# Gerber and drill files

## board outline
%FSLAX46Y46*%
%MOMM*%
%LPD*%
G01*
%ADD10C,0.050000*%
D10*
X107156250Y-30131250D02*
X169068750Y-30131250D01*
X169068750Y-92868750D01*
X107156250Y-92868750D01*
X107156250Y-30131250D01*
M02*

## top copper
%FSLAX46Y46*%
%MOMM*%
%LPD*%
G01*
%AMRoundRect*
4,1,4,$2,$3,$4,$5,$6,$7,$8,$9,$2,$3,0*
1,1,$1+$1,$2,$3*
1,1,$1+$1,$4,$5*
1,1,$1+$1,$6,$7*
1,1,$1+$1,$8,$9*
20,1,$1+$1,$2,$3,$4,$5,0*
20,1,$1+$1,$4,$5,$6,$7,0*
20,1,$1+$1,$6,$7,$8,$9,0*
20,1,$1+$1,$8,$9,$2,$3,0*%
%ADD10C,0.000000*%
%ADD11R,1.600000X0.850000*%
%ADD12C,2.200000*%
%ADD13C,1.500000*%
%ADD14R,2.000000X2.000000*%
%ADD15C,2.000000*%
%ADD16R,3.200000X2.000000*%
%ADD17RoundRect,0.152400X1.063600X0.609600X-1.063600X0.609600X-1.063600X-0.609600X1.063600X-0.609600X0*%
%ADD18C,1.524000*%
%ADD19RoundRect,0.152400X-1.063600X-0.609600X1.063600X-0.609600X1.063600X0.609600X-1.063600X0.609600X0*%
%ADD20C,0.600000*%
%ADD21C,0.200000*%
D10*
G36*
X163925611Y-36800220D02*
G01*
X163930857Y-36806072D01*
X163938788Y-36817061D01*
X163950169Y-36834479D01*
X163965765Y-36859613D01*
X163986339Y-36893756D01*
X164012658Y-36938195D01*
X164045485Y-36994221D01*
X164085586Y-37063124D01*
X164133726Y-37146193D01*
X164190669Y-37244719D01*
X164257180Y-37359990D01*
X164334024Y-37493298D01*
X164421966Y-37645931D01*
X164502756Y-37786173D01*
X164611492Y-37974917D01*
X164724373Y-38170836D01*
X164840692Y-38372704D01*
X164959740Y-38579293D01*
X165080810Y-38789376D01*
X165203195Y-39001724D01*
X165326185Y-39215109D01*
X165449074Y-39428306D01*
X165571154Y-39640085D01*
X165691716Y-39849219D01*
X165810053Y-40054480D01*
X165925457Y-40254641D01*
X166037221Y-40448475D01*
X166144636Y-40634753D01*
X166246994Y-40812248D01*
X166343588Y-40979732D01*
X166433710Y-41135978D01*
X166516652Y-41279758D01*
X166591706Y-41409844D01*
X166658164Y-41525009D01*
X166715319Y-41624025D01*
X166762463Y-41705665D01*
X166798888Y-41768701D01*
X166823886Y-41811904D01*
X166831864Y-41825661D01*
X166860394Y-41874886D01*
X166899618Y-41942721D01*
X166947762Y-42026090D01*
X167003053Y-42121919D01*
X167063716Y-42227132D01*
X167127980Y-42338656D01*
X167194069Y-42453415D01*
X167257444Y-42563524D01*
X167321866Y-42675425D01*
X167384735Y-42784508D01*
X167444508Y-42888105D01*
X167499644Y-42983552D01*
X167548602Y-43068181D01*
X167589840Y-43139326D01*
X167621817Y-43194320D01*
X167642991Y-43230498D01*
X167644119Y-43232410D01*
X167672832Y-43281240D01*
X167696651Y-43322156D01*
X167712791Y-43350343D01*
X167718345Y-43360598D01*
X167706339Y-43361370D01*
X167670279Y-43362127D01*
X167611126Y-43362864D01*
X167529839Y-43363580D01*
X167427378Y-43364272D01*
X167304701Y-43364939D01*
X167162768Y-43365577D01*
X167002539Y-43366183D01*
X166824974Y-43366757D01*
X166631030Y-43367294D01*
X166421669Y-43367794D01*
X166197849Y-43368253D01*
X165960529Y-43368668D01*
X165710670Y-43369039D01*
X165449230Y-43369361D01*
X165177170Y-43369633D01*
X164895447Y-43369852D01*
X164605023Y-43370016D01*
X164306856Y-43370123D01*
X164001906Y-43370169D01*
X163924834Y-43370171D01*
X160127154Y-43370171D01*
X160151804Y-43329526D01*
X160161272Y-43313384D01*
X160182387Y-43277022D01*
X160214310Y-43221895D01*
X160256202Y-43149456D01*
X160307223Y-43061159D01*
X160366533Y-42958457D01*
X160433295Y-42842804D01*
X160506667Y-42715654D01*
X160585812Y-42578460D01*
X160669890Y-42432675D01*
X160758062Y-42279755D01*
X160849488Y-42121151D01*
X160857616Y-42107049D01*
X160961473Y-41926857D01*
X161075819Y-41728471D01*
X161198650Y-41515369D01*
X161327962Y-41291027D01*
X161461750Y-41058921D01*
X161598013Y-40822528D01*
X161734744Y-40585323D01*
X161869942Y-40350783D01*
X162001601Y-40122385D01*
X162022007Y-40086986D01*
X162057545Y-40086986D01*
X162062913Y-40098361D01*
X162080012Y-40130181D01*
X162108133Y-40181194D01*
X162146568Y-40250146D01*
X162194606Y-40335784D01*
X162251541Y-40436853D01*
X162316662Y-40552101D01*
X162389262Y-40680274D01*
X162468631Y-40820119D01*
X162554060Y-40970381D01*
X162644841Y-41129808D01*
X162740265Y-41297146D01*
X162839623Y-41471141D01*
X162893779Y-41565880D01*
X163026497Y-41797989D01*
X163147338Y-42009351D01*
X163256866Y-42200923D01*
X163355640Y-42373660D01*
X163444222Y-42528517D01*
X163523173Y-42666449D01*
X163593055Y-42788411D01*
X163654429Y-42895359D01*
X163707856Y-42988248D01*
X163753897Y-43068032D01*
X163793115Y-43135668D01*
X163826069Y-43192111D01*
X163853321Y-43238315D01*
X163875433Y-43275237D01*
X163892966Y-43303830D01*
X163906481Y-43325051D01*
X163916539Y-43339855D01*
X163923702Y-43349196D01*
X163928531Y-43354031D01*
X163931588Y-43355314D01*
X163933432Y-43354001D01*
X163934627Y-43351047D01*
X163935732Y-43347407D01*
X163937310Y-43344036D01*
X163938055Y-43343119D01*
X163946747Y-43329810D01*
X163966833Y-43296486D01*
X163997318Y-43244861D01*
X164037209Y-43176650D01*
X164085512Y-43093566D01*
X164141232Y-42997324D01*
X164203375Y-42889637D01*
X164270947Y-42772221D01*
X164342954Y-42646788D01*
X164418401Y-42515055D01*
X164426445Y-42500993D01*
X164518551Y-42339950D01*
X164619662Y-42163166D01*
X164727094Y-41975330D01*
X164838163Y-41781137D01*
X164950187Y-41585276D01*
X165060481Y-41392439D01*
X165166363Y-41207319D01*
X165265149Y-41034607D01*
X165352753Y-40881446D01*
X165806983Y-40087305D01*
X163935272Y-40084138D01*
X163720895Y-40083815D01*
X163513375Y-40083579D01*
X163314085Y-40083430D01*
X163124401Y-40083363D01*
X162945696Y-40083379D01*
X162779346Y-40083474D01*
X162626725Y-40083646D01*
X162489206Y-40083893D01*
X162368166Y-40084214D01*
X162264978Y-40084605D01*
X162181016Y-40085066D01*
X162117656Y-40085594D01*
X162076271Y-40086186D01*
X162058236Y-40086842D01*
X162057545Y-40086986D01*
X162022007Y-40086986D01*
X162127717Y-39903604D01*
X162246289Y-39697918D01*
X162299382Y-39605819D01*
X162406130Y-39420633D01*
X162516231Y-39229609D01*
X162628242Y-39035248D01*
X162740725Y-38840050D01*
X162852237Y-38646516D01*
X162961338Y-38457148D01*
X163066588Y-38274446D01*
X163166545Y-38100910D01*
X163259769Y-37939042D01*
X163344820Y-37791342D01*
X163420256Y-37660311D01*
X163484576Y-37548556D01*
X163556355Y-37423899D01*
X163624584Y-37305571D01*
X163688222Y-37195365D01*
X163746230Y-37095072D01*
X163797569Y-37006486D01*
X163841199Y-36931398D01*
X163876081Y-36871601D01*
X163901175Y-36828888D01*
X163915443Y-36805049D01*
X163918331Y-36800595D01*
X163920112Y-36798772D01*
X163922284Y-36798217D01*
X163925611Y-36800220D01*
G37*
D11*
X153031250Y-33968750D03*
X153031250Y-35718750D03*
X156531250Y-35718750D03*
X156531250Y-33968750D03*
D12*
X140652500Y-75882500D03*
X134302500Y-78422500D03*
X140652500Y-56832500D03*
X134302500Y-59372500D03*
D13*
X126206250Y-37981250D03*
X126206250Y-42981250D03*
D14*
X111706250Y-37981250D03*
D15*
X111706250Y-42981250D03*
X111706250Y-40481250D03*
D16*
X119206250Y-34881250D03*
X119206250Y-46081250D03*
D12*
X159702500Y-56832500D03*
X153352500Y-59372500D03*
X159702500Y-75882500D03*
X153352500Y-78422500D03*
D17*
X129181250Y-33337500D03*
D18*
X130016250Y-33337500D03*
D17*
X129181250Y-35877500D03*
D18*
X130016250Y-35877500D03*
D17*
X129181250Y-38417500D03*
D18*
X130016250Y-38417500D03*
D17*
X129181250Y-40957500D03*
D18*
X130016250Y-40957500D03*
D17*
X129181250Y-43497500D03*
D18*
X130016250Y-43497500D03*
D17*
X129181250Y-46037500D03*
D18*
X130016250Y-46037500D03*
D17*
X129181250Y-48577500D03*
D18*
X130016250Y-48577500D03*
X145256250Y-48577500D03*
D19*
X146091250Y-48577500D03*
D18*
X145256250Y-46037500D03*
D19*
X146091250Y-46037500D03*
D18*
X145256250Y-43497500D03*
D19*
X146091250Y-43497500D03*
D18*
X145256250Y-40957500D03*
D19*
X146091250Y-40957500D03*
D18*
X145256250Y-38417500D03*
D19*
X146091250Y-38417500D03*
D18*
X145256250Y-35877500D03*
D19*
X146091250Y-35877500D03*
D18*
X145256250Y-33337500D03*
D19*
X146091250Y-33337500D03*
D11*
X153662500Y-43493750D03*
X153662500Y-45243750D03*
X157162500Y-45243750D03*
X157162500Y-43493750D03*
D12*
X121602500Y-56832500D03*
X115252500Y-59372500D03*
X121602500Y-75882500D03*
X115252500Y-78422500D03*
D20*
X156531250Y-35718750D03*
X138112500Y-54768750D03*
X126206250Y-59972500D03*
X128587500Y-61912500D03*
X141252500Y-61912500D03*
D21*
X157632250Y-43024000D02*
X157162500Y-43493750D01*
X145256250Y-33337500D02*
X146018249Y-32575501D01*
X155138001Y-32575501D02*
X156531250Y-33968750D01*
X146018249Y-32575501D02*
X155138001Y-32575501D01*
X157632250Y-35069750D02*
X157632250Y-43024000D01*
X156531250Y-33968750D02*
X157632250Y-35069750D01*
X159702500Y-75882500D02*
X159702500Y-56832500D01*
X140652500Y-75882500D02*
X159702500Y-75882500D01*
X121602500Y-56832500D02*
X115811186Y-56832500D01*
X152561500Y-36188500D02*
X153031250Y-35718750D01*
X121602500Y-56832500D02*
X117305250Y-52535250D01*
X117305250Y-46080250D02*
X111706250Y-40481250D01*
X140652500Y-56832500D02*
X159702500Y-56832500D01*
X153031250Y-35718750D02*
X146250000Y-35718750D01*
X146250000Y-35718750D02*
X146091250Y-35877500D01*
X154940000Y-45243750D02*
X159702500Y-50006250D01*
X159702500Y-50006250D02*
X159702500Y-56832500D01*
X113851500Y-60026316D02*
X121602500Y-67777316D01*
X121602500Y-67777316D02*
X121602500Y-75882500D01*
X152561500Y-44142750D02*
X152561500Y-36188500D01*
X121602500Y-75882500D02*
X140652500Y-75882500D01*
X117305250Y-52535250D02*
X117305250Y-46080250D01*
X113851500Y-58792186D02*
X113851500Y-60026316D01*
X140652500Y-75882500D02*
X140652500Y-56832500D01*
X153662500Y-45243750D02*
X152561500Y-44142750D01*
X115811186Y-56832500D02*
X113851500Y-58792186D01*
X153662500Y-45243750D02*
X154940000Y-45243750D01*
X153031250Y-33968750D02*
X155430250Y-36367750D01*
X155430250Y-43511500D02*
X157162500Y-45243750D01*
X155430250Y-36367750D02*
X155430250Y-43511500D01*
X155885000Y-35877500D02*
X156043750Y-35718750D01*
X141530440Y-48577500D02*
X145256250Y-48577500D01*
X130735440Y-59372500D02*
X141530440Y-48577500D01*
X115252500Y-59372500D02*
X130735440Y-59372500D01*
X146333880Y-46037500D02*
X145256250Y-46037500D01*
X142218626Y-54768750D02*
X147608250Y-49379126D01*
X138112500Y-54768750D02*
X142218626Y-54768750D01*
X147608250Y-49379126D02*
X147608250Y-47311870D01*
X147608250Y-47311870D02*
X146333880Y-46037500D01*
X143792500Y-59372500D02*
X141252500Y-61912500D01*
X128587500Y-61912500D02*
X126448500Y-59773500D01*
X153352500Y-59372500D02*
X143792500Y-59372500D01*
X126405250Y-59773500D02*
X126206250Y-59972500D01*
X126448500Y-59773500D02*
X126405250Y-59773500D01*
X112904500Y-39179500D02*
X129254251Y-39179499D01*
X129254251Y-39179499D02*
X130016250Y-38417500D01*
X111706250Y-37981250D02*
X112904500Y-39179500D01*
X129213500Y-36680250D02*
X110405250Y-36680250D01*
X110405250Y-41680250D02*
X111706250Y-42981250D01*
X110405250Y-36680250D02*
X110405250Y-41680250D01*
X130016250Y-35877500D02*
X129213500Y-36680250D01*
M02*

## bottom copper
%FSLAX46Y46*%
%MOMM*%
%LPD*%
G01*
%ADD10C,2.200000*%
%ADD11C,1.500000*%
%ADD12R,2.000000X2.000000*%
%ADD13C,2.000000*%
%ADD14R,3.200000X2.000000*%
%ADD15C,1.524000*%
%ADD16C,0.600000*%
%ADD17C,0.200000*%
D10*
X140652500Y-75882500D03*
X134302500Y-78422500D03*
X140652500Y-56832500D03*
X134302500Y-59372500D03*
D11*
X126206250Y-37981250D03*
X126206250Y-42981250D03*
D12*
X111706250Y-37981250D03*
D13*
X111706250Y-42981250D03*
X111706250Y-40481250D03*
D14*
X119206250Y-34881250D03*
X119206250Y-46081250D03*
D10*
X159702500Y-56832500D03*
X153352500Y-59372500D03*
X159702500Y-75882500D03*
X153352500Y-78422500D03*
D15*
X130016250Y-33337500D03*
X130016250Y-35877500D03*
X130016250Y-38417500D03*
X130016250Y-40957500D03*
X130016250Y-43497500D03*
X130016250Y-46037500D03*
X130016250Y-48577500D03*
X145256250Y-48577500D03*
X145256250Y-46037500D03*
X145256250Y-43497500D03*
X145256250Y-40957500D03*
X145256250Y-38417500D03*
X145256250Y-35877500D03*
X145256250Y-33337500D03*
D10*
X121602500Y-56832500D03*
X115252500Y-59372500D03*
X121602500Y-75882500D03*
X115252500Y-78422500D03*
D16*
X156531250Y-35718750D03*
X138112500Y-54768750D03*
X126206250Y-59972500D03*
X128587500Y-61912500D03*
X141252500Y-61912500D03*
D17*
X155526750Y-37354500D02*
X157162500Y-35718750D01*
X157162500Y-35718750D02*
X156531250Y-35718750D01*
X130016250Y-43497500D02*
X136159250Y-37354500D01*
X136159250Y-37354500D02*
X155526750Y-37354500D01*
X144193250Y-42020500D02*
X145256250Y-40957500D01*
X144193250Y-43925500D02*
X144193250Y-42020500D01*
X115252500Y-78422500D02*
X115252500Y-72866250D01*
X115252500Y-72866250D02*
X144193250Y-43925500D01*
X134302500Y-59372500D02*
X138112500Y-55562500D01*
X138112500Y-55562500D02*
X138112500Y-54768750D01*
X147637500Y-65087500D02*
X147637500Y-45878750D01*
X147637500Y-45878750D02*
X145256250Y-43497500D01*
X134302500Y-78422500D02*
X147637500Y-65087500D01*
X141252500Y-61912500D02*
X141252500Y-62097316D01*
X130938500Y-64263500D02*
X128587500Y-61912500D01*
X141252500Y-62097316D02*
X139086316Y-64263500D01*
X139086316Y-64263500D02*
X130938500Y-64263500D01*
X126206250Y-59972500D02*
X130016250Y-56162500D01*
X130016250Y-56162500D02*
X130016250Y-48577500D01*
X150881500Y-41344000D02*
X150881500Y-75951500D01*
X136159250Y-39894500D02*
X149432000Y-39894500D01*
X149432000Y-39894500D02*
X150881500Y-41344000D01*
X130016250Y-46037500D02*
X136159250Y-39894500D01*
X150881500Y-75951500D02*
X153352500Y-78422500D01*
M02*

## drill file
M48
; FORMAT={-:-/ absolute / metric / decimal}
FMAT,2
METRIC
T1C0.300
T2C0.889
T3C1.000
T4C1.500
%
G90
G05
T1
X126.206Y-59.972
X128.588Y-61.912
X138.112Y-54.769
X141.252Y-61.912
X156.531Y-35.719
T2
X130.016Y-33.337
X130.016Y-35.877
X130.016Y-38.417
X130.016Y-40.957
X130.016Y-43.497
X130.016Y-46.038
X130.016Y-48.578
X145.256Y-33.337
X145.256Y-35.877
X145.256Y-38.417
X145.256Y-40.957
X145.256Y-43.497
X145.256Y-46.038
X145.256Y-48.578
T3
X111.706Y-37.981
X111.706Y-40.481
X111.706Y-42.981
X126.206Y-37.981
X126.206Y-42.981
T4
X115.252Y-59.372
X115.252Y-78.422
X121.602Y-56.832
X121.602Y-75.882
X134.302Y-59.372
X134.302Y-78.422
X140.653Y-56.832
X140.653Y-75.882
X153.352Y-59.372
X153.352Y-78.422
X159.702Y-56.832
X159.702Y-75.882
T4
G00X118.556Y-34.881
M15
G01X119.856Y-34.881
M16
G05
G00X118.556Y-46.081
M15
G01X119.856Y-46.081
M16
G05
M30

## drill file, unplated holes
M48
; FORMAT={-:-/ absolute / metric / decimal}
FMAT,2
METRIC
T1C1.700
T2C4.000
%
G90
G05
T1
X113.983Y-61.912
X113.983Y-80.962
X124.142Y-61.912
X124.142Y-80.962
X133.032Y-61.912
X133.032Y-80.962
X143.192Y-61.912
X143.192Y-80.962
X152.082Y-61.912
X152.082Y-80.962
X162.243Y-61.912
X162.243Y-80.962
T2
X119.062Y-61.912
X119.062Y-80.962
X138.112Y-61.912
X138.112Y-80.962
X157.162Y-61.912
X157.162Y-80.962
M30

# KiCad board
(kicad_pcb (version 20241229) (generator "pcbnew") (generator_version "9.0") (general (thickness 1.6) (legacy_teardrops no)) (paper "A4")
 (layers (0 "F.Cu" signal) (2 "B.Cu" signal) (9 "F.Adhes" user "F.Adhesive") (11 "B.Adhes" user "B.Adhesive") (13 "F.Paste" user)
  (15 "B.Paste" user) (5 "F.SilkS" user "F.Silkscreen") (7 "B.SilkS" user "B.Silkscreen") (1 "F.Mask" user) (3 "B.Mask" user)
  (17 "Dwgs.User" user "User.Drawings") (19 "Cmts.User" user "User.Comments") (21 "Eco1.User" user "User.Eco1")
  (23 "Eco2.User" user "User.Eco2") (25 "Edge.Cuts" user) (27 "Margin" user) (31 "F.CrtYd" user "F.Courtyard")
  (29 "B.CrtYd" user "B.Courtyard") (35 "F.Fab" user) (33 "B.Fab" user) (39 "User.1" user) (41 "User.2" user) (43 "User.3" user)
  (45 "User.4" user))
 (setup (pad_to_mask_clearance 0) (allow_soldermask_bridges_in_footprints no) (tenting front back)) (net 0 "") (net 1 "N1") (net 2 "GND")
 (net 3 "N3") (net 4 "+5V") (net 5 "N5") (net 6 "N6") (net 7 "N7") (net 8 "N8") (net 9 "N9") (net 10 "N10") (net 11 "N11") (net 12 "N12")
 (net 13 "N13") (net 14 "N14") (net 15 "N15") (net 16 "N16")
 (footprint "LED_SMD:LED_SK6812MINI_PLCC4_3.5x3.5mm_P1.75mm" (layer "F.Cu") (at 154.78125 34.84375)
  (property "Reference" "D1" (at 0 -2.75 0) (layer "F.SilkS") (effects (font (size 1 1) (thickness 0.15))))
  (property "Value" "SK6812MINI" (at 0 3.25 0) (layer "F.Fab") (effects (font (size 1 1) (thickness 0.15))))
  (pad "1" smd rect (at -1.75 -0.875) (size 1.6 0.85) (layers "F.Cu" "F.Mask" "F.Paste") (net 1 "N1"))
  (pad "2" smd rect (at -1.75 0.875) (size 1.6 0.85) (layers "F.Cu" "F.Mask" "F.Paste") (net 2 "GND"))
  (pad "3" smd rect (at 1.75 0.875) (size 1.6 0.85) (layers "F.Cu" "F.Mask" "F.Paste") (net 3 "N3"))
  (pad "4" smd rect (at 1.75 -0.875) (size 1.6 0.85) (layers "F.Cu" "F.Mask" "F.Paste") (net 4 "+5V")))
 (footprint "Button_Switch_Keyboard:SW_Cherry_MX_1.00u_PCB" (layer "F.Cu") (at 140.6525 75.8825)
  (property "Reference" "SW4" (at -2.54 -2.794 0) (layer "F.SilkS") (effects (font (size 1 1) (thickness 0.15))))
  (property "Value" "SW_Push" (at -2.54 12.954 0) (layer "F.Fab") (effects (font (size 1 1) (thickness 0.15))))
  (pad "" np_thru_hole circle (at -7.62 5.08) (size 1.7 1.7) (drill 1.7) (layers "*.Cu" "*.Mask"))
  (pad "" np_thru_hole circle (at -2.54 5.08) (size 4 4) (drill 4) (layers "*.Cu" "*.Mask"))
  (pad "" np_thru_hole circle (at 2.54 5.08) (size 1.7 1.7) (drill 1.7) (layers "*.Cu" "*.Mask"))
  (pad "1" thru_hole circle (at 0 0) (size 2.2 2.2) (drill 1.5) (layers "*.Cu" "*.Mask") (remove_unused_layers no) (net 2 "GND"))
  (pad "2" thru_hole circle (at -6.35 2.54) (size 2.2 2.2) (drill 1.5) (layers "*.Cu" "*.Mask") (remove_unused_layers no) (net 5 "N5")))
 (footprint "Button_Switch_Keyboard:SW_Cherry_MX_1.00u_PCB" (layer "F.Cu") (at 140.6525 56.8325)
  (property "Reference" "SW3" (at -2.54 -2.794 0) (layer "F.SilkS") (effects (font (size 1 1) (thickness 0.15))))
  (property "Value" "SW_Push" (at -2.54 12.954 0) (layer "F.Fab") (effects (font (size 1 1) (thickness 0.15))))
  (pad "" np_thru_hole circle (at -7.62 5.08) (size 1.7 1.7) (drill 1.7) (layers "*.Cu" "*.Mask"))
  (pad "" np_thru_hole circle (at -2.54 5.08) (size 4 4) (drill 4) (layers "*.Cu" "*.Mask"))
  (pad "" np_thru_hole circle (at 2.54 5.08) (size 1.7 1.7) (drill 1.7) (layers "*.Cu" "*.Mask"))
  (pad "1" thru_hole circle (at 0 0) (size 2.2 2.2) (drill 1.5) (layers "*.Cu" "*.Mask") (remove_unused_layers no) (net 2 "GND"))
  (pad "2" thru_hole circle (at -6.35 2.54) (size 2.2 2.2) (drill 1.5) (layers "*.Cu" "*.Mask") (remove_unused_layers no) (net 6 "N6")))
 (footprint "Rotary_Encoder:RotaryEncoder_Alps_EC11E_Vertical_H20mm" (layer "F.Cu") (at 111.70625 37.98125)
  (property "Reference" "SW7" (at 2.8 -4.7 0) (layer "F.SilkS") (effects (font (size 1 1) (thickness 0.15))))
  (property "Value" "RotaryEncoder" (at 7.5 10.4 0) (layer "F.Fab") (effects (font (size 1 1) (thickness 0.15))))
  (pad "" thru_hole circle (at 14.5 0) (size 1.5 1.5) (drill 1) (layers "*.Cu" "*.Mask") (remove_unused_layers no))
  (pad "" thru_hole circle (at 14.5 5) (size 1.5 1.5) (drill 1) (layers "*.Cu" "*.Mask") (remove_unused_layers no))
  (pad "A" thru_hole rect (at 0 0) (size 2 2) (drill 1) (layers "*.Cu" "*.Mask") (remove_unused_layers no) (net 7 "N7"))
  (pad "B" thru_hole circle (at 0 5) (size 2 2) (drill 1) (layers "*.Cu" "*.Mask") (remove_unused_layers no) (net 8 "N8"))
  (pad "C" thru_hole circle (at 0 2.5) (size 2 2) (drill 1) (layers "*.Cu" "*.Mask") (remove_unused_layers no) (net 2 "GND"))
  (pad "MP" thru_hole rect (at 7.5 -3.1) (size 3.2 2) (drill oval 2.8 1.5) (layers "*.Cu" "*.Mask") (remove_unused_layers no))
  (pad "MP" thru_hole rect (at 7.5 8.1) (size 3.2 2) (drill oval 2.8 1.5) (layers "*.Cu" "*.Mask") (remove_unused_layers no)))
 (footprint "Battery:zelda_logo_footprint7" (layer "F.Cu") (at 164.30625 40.48125)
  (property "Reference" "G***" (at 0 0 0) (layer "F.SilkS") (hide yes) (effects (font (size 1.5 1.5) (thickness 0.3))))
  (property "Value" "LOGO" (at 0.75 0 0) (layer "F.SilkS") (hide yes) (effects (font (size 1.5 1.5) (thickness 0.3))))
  (fp_poly
   (pts (xy -0.380639 -3.68103) (xy -0.375393 -3.675178) (xy -0.367462 -3.664189) (xy -0.356081 -3.646771) (xy -0.340485 -3.621637)
    (xy -0.319911 -3.587494) (xy -0.293592 -3.543055) (xy -0.260765 -3.487029) (xy -0.220664 -3.418126) (xy -0.172524 -3.335057)
    (xy -0.115581 -3.236531) (xy -0.04907 -3.12126) (xy 0.027774 -2.987952) (xy 0.115716 -2.835319) (xy 0.196506 -2.695077)
    (xy 0.305242 -2.506333) (xy 0.418123 -2.310414) (xy 0.534442 -2.108546) (xy 0.65349 -1.901957) (xy 0.77456 -1.691874)
    (xy 0.896945 -1.479526) (xy 1.019935 -1.266141) (xy 1.142824 -1.052944) (xy 1.264904 -0.841165) (xy 1.385466 -0.632031)
    (xy 1.503803 -0.42677) (xy 1.619207 -0.226609) (xy 1.730971 -0.032775) (xy 1.838386 0.153503) (xy 1.940744 0.330998)
    (xy 2.037338 0.498482) (xy 2.12746 0.654728) (xy 2.210402 0.798508) (xy 2.285456 0.928594) (xy 2.351914 1.043759) (xy 2.409069 1.142775)
    (xy 2.456213 1.224415) (xy 2.492638 1.287451) (xy 2.517636 1.330654) (xy 2.525614 1.344411) (xy 2.554144 1.393636)
    (xy 2.593368 1.461471) (xy 2.641512 1.54484) (xy 2.696803 1.640669) (xy 2.757466 1.745882) (xy 2.82173 1.857406) (xy 2.887819 1.972165)
    (xy 2.951194 2.082274) (xy 3.015616 2.194175) (xy 3.078485 2.303258) (xy 3.138258 2.406855) (xy 3.193394 2.502302)
    (xy 3.242352 2.586931) (xy 3.28359 2.658076) (xy 3.315567 2.71307) (xy 3.336741 2.749248) (xy 3.337869 2.75116) (xy 3.366582 2.79999)
    (xy 3.390401 2.840906) (xy 3.406541 2.869093) (xy 3.412095 2.879348) (xy 3.400089 2.88012) (xy 3.364029 2.880877) (xy 3.304876 2.881614)
    (xy 3.223589 2.88233) (xy 3.121128 2.883022) (xy 2.998451 2.883689) (xy 2.856518 2.884327) (xy 2.696289 2.884933) (xy 2.518724 2.885507)
    (xy 2.32478 2.886044) (xy 2.115419 2.886544) (xy 1.891599 2.887003) (xy 1.654279 2.887418) (xy 1.40442 2.887789) (xy 1.14298 2.888111)
    (xy 0.87092 2.888383) (xy 0.589197 2.888602) (xy 0.298773 2.888766) (xy 0.000606 2.888873) (xy -0.304344 2.888919)
    (xy -0.381416 2.888921) (xy -4.179096 2.888921) (xy -4.154446 2.848276) (xy -4.144978 2.832134) (xy -4.123863 2.795772)
    (xy -4.09194 2.740645) (xy -4.050048 2.668206) (xy -3.999027 2.579909) (xy -3.939717 2.477207) (xy -3.872955 2.361554)
    (xy -3.799583 2.234404) (xy -3.720438 2.09721) (xy -3.63636 1.951425) (xy -3.548188 1.798505) (xy -3.456762 1.639901)
    (xy -3.448634 1.625799) (xy -3.344777 1.445607) (xy -3.230431 1.247221) (xy -3.1076 1.034119) (xy -2.978288 0.809777)
    (xy -2.8445 0.577671) (xy -2.708237 0.341278) (xy -2.571506 0.104073) (xy -2.436308 -0.130467) (xy -2.304649 -0.358865)
    (xy -2.284243 -0.394264) (xy -2.248705 -0.394264) (xy -2.243337 -0.382889) (xy -2.226238 -0.351069) (xy -2.198117 -0.300056)
    (xy -2.159682 -0.231104) (xy -2.111644 -0.145466) (xy -2.054709 -0.044397) (xy -1.989588 0.070851) (xy -1.916988 0.199024)
    (xy -1.837619 0.338869) (xy -1.75219 0.489131) (xy -1.661409 0.648558) (xy -1.565985 0.815896) (xy -1.466627 0.989891)
    (xy -1.412471 1.08463) (xy -1.279753 1.316739) (xy -1.158912 1.528101) (xy -1.049384 1.719673) (xy -0.95061 1.89241)
    (xy -0.862028 2.047267) (xy -0.783077 2.185199) (xy -0.713195 2.307161) (xy -0.651821 2.414109) (xy -0.598394 2.506998)
    (xy -0.552353 2.586782) (xy -0.513135 2.654418) (xy -0.480181 2.710861) (xy -0.452929 2.757065) (xy -0.430817 2.793987)
    (xy -0.413284 2.82258) (xy -0.399769 2.843801) (xy -0.389711 2.858605) (xy -0.382548 2.867946) (xy -0.377719 2.872781)
    (xy -0.374662 2.874064) (xy -0.372818 2.872751) (xy -0.371623 2.869797) (xy -0.370518 2.866157) (xy -0.36894 2.862786)
    (xy -0.368195 2.861869) (xy -0.359503 2.84856) (xy -0.339417 2.815236) (xy -0.308932 2.763611) (xy -0.269041 2.6954)
    (xy -0.220738 2.612316) (xy -0.165018 2.516074) (xy -0.102875 2.408387) (xy -0.035303 2.290971) (xy 0.036704 2.165538)
    (xy 0.112151 2.033805) (xy 0.120195 2.019743) (xy 0.212301 1.8587) (xy 0.313412 1.681916) (xy 0.420844 1.49408) (xy 0.531913 1.299887)
    (xy 0.643937 1.104026) (xy 0.754231 0.911189) (xy 0.860113 0.726069) (xy 0.958899 0.553357) (xy 1.046503 0.400196)
    (xy 1.500733 -0.393945) (xy -0.370978 -0.397112) (xy -0.585355 -0.397435) (xy -0.792875 -0.397671) (xy -0.992165 -0.39782)
    (xy -1.181849 -0.397887) (xy -1.360554 -0.397871) (xy -1.526904 -0.397776) (xy -1.679525 -0.397604) (xy -1.817044 -0.397357)
    (xy -1.938084 -0.397036) (xy -2.041272 -0.396645) (xy -2.125234 -0.396184) (xy -2.188594 -0.395656) (xy -2.229979 -0.395064)
    (xy -2.248014 -0.394408) (xy -2.248705 -0.394264) (xy -2.284243 -0.394264) (xy -2.178533 -0.577646) (xy -2.059961 -0.783332)
    (xy -2.006868 -0.875431) (xy -1.90012 -1.060617) (xy -1.790019 -1.251641) (xy -1.678008 -1.446002) (xy -1.565525 -1.6412)
    (xy -1.454013 -1.834734) (xy -1.344912 -2.024102) (xy -1.239662 -2.206804) (xy -1.139705 -2.38034) (xy -1.046481 -2.542208)
    (xy -0.96143 -2.689908) (xy -0.885994 -2.820939) (xy -0.821674 -2.932694) (xy -0.749895 -3.057351) (xy -0.681666 -3.175679)
    (xy -0.618028 -3.285885) (xy -0.56002 -3.386178) (xy -0.508681 -3.474764) (xy -0.465051 -3.549852) (xy -0.430169 -3.609649)
    (xy -0.405075 -3.652362) (xy -0.390807 -3.676201) (xy -0.387919 -3.680655) (xy -0.386138 -3.682478) (xy -0.383966 -3.683033))
   (stroke (width 0) (type solid)) (fill yes) (layer "F.Cu")))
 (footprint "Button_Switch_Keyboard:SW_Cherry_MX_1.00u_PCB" (layer "F.Cu") (at 159.7025 56.8325)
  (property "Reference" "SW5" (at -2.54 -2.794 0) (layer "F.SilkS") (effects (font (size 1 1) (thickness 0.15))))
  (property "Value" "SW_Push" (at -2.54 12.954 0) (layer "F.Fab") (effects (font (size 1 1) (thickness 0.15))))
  (pad "" np_thru_hole circle (at -7.62 5.08) (size 1.7 1.7) (drill 1.7) (layers "*.Cu" "*.Mask"))
  (pad "" np_thru_hole circle (at -2.54 5.08) (size 4 4) (drill 4) (layers "*.Cu" "*.Mask"))
  (pad "" np_thru_hole circle (at 2.54 5.08) (size 1.7 1.7) (drill 1.7) (layers "*.Cu" "*.Mask"))
  (pad "1" thru_hole circle (at 0 0) (size 2.2 2.2) (drill 1.5) (layers "*.Cu" "*.Mask") (remove_unused_layers no) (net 2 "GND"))
  (pad "2" thru_hole circle (at -6.35 2.54) (size 2.2 2.2) (drill 1.5) (layers "*.Cu" "*.Mask") (remove_unused_layers no) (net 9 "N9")))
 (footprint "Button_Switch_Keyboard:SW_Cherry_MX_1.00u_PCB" (layer "F.Cu") (at 159.7025 75.8825)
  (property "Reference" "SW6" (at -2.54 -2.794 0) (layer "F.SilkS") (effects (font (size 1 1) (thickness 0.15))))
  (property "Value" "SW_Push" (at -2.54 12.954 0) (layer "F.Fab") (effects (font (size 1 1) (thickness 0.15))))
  (pad "" np_thru_hole circle (at -7.62 5.08) (size 1.7 1.7) (drill 1.7) (layers "*.Cu" "*.Mask"))
  (pad "" np_thru_hole circle (at -2.54 5.08) (size 4 4) (drill 4) (layers "*.Cu" "*.Mask"))
  (pad "" np_thru_hole circle (at 2.54 5.08) (size 1.7 1.7) (drill 1.7) (layers "*.Cu" "*.Mask"))
  (pad "1" thru_hole circle (at 0 0) (size 2.2 2.2) (drill 1.5) (layers "*.Cu" "*.Mask") (remove_unused_layers no) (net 2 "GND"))
  (pad "2" thru_hole circle (at -6.35 2.54) (size 2.2 2.2) (drill 1.5) (layers "*.Cu" "*.Mask") (remove_unused_layers no) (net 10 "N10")))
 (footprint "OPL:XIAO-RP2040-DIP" (layer "F.Cu") (at 137.63625 40.9575)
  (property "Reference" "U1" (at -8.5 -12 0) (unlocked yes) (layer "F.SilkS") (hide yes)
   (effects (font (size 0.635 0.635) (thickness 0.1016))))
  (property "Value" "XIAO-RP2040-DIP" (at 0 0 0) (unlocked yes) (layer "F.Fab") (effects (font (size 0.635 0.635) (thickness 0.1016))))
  (pad "1" smd roundrect (at -8.455 -7.62 180) (size 2.432 1.524) (layers "F.Cu" "F.Mask") (roundrect_rratio 0.1) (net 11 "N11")
   (thermal_bridge_angle 45))
  (pad "1" thru_hole circle (at -7.62 -7.62 180) (size 1.524 1.524) (drill 0.889) (layers "*.Cu" "*.Mask") (remove_unused_layers no)
   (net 11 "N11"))
  (pad "2" smd roundrect (at -8.455 -5.08 180) (size 2.432 1.524) (layers "F.Cu" "F.Mask") (roundrect_rratio 0.1) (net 8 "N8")
   (thermal_bridge_angle 45))
  (pad "2" thru_hole circle (at -7.62 -5.08 180) (size 1.524 1.524) (drill 0.889) (layers "*.Cu" "*.Mask") (remove_unused_layers no)
   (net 8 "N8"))
  (pad "3" smd roundrect (at -8.455 -2.54 180) (size 2.432 1.524) (layers "F.Cu" "F.Mask") (roundrect_rratio 0.1) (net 7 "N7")
   (thermal_bridge_angle 45))
  (pad "3" thru_hole circle (at -7.62 -2.54 180) (size 1.524 1.524) (drill 0.889) (layers "*.Cu" "*.Mask") (remove_unused_layers no)
   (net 7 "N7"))
  (pad "4" smd roundrect (at -8.455 0 180) (size 2.432 1.524) (layers "F.Cu" "F.Mask") (roundrect_rratio 0.1) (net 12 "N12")
   (thermal_bridge_angle 45))
  (pad "4" thru_hole circle (at -7.62 0 180) (size 1.524 1.524) (drill 0.889) (layers "*.Cu" "*.Mask") (remove_unused_layers no)
   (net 12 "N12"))
  (pad "5" smd roundrect (at -8.455 2.54 180) (size 2.432 1.524) (layers "F.Cu" "F.Mask") (roundrect_rratio 0.1) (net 3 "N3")
   (thermal_bridge_angle 45))
  (pad "5" thru_hole circle (at -7.62 2.54 180) (size 1.524 1.524) (drill 0.889) (layers "*.Cu" "*.Mask") (remove_unused_layers no)
   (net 3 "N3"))
  (pad "6" smd roundrect (at -8.455 5.08 180) (size 2.432 1.524) (layers "F.Cu" "F.Mask") (roundrect_rratio 0.1) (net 10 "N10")
   (thermal_bridge_angle 45))
  (pad "6" thru_hole circle (at -7.62 5.08 180) (size 1.524 1.524) (drill 0.889) (layers "*.Cu" "*.Mask") (remove_unused_layers no)
   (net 10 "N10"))
  (pad "7" smd roundrect (at -8.455 7.62 180) (size 2.432 1.524) (layers "F.Cu" "F.Mask") (roundrect_rratio 0.1) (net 9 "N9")
   (thermal_bridge_angle 45))
  (pad "7" thru_hole circle (at -7.62 7.62 180) (size 1.524 1.524) (drill 0.889) (layers "*.Cu" "*.Mask") (remove_unused_layers no)
   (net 9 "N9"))
  (pad "8" thru_hole circle (at 7.62 7.62) (size 1.524 1.524) (drill 0.889) (layers "*.Cu" "*.Mask") (remove_unused_layers no)
   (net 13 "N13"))
  (pad "8" smd roundrect (at 8.455 7.62) (size 2.432 1.524) (layers "F.Cu" "F.Mask") (roundrect_rratio 0.1) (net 13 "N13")
   (thermal_bridge_angle 45))
  (pad "9" thru_hole circle (at 7.62 5.08) (size 1.524 1.524) (drill 0.889) (layers "*.Cu" "*.Mask") (remove_unused_layers no) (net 6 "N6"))
  (pad "9" smd roundrect (at 8.455 5.08) (size 2.432 1.524) (layers "F.Cu" "F.Mask") (roundrect_rratio 0.1) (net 6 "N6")
   (thermal_bridge_angle 45))
  (pad "10" thru_hole circle (at 7.62 2.54) (size 1.524 1.524) (drill 0.889) (layers "*.Cu" "*.Mask") (remove_unused_layers no) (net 5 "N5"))
  (pad "10" smd roundrect (at 8.455 2.54) (size 2.432 1.524) (layers "F.Cu" "F.Mask") (roundrect_rratio 0.1) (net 5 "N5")
   (thermal_bridge_angle 45))
  (pad "11" thru_hole circle (at 7.62 0) (size 1.524 1.524) (drill 0.889) (layers "*.Cu" "*.Mask") (remove_unused_layers no) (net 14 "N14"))
  (pad "11" smd roundrect (at 8.455 0) (size 2.432 1.524) (layers "F.Cu" "F.Mask") (roundrect_rratio 0.1) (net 14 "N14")
   (thermal_bridge_angle 45))
  (pad "12" thru_hole circle (at 7.62 -2.54) (size 1.524 1.524) (drill 0.889) (layers "*.Cu" "*.Mask") (remove_unused_layers no)
   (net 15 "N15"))
  (pad "12" smd roundrect (at 8.455 -2.54) (size 2.432 1.524) (layers "F.Cu" "F.Mask") (roundrect_rratio 0.1) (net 15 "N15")
   (thermal_bridge_angle 45))
  (pad "13" thru_hole circle (at 7.62 -5.08) (size 1.524 1.524) (drill 0.889) (layers "*.Cu" "*.Mask") (remove_unused_layers no)
   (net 2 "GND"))
  (pad "13" smd roundrect (at 8.455 -5.08) (size 2.432 1.524) (layers "F.Cu" "F.Mask") (roundrect_rratio 0.1) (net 2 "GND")
   (thermal_bridge_angle 45))
  (pad "14" thru_hole circle (at 7.62 -7.62) (size 1.524 1.524) (drill 0.889) (layers "*.Cu" "*.Mask") (remove_unused_layers no)
   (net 4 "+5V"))
  (pad "14" smd roundrect (at 8.455 -7.62) (size 2.432 1.524) (layers "F.Cu" "F.Mask") (roundrect_rratio 0.1) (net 4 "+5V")
   (thermal_bridge_angle 45)))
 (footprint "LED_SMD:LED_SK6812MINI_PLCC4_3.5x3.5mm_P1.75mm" (layer "F.Cu") (at 155.4125 44.36875)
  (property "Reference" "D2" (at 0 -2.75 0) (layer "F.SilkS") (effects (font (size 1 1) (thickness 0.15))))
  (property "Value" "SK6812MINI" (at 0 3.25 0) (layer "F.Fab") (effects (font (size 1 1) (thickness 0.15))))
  (pad "1" smd rect (at -1.75 -0.875) (size 1.6 0.85) (layers "F.Cu" "F.Mask" "F.Paste") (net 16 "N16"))
  (pad "2" smd rect (at -1.75 0.875) (size 1.6 0.85) (layers "F.Cu" "F.Mask" "F.Paste") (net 2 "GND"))
  (pad "3" smd rect (at 1.75 0.875) (size 1.6 0.85) (layers "F.Cu" "F.Mask" "F.Paste") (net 1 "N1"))
  (pad "4" smd rect (at 1.75 -0.875) (size 1.6 0.85) (layers "F.Cu" "F.Mask" "F.Paste") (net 4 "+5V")))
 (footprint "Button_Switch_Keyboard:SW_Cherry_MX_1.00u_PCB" (layer "F.Cu") (at 121.6025 56.8325)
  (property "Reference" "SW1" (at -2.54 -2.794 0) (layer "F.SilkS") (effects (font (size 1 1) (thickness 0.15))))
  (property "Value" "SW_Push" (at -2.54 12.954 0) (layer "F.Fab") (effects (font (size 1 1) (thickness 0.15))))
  (pad "" np_thru_hole circle (at -7.62 5.08) (size 1.7 1.7) (drill 1.7) (layers "*.Cu" "*.Mask"))
  (pad "" np_thru_hole circle (at -2.54 5.08) (size 4 4) (drill 4) (layers "*.Cu" "*.Mask"))
  (pad "" np_thru_hole circle (at 2.54 5.08) (size 1.7 1.7) (drill 1.7) (layers "*.Cu" "*.Mask"))
  (pad "1" thru_hole circle (at 0 0) (size 2.2 2.2) (drill 1.5) (layers "*.Cu" "*.Mask") (remove_unused_layers no) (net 2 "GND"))
  (pad "2" thru_hole circle (at -6.35 2.54) (size 2.2 2.2) (drill 1.5) (layers "*.Cu" "*.Mask") (remove_unused_layers no) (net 13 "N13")))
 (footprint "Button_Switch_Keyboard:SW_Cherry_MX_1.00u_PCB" (layer "F.Cu") (at 121.6025 75.8825)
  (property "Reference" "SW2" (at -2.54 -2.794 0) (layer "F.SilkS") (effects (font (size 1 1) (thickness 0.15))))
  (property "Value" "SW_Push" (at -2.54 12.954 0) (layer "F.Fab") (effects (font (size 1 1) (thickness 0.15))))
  (pad "" np_thru_hole circle (at -7.62 5.08) (size 1.7 1.7) (drill 1.7) (layers "*.Cu" "*.Mask"))
  (pad "" np_thru_hole circle (at -2.54 5.08) (size 4 4) (drill 4) (layers "*.Cu" "*.Mask"))
  (pad "" np_thru_hole circle (at 2.54 5.08) (size 1.7 1.7) (drill 1.7) (layers "*.Cu" "*.Mask"))
  (pad "1" thru_hole circle (at 0 0) (size 2.2 2.2) (drill 1.5) (layers "*.Cu" "*.Mask") (remove_unused_layers no) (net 2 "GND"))
  (pad "2" thru_hole circle (at -6.35 2.54) (size 2.2 2.2) (drill 1.5) (layers "*.Cu" "*.Mask") (remove_unused_layers no) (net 14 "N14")))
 (gr_rect (start 107.15625 30.13125) (end 169.06875 92.86875) (stroke (width 0.05) (type default)) (fill no) (layer "Edge.Cuts"))
 (segment (start 157.63225 43.024) (end 157.1625 43.49375) (width 0.2) (layer "F.Cu") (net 4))
 (segment (start 145.25625 33.3375) (end 146.018249 32.575501) (width 0.2) (layer "F.Cu") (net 4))
 (segment (start 155.138001 32.575501) (end 156.53125 33.96875) (width 0.2) (layer "F.Cu") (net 4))
 (segment (start 146.018249 32.575501) (end 155.138001 32.575501) (width 0.2) (layer "F.Cu") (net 4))
 (segment (start 157.63225 35.06975) (end 157.63225 43.024) (width 0.2) (layer "F.Cu") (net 4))
 (segment (start 156.53125 33.96875) (end 157.63225 35.06975) (width 0.2) (layer "F.Cu") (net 4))
 (segment (start 159.7025 75.8825) (end 159.7025 56.8325) (width 0.2) (layer "F.Cu") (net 2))
 (segment (start 140.6525 75.8825) (end 159.7025 75.8825) (width 0.2) (layer "F.Cu") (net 2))
 (segment (start 121.6025 56.8325) (end 115.811186 56.8325) (width 0.2) (layer "F.Cu") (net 2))
 (segment (start 152.5615 36.1885) (end 153.03125 35.71875) (width 0.2) (layer "F.Cu") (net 2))
 (segment (start 121.6025 56.8325) (end 117.30525 52.53525) (width 0.2) (layer "F.Cu") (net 2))
 (segment (start 117.30525 46.08025) (end 111.70625 40.48125) (width 0.2) (layer "F.Cu") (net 2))
 (segment (start 140.6525 56.8325) (end 159.7025 56.8325) (width 0.2) (layer "F.Cu") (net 2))
 (segment (start 153.03125 35.71875) (end 146.25 35.71875) (width 0.2) (layer "F.Cu") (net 2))
 (segment (start 146.25 35.71875) (end 146.09125 35.8775) (width 0.2) (layer "F.Cu") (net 2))
 (segment (start 154.94 45.24375) (end 159.7025 50.00625) (width 0.2) (layer "F.Cu") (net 2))
 (segment (start 159.7025 50.00625) (end 159.7025 56.8325) (width 0.2) (layer "F.Cu") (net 2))
 (segment (start 113.8515 60.026316) (end 121.6025 67.777316) (width 0.2) (layer "F.Cu") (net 2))
 (segment (start 121.6025 67.777316) (end 121.6025 75.8825) (width 0.2) (layer "F.Cu") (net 2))
 (segment (start 152.5615 44.14275) (end 152.5615 36.1885) (width 0.2) (layer "F.Cu") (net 2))
 (segment (start 121.6025 75.8825) (end 140.6525 75.8825) (width 0.2) (layer "F.Cu") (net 2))
 (segment (start 117.30525 52.53525) (end 117.30525 46.08025) (width 0.2) (layer "F.Cu") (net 2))
 (segment (start 113.8515 58.792186) (end 113.8515 60.026316) (width 0.2) (layer "F.Cu") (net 2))
 (segment (start 140.6525 75.8825) (end 140.6525 56.8325) (width 0.2) (layer "F.Cu") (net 2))
 (segment (start 153.6625 45.24375) (end 152.5615 44.14275) (width 0.2) (layer "F.Cu") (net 2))
 (segment (start 115.811186 56.8325) (end 113.8515 58.792186) (width 0.2) (layer "F.Cu") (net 2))
 (segment (start 153.6625 45.24375) (end 154.94 45.24375) (width 0.2) (layer "F.Cu") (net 2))
 (segment (start 153.03125 33.96875) (end 155.43025 36.36775) (width 0.2) (layer "F.Cu") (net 1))
 (segment (start 155.43025 43.5115) (end 157.1625 45.24375) (width 0.2) (layer "F.Cu") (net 1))
 (segment (start 155.43025 36.36775) (end 155.43025 43.5115) (width 0.2) (layer "F.Cu") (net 1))
 (segment (start 155.885 35.8775) (end 156.04375 35.71875) (width 0.2) (layer "F.Cu") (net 3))
 (via (at 156.53125 35.71875) (size 0.6) (drill 0.3) (layers "F.Cu" "B.Cu") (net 3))
 (segment (start 155.52675 37.3545) (end 157.1625 35.71875) (width 0.2) (layer "B.Cu") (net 3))
 (segment (start 157.1625 35.71875) (end 156.53125 35.71875) (width 0.2) (layer "B.Cu") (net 3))
 (segment (start 130.01625 43.4975) (end 136.15925 37.3545) (width 0.2) (layer "B.Cu") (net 3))
 (segment (start 136.15925 37.3545) (end 155.52675 37.3545) (width 0.2) (layer "B.Cu") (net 3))
 (segment (start 141.53044 48.5775) (end 145.25625 48.5775) (width 0.2) (layer "F.Cu") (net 13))
 (segment (start 130.73544 59.3725) (end 141.53044 48.5775) (width 0.2) (layer "F.Cu") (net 13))
 (segment (start 115.2525 59.3725) (end 130.73544 59.3725) (width 0.2) (layer "F.Cu") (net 13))
 (segment (start 144.19325 42.0205) (end 145.25625 40.9575) (width 0.2) (layer "B.Cu") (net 14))
 (segment (start 144.19325 43.9255) (end 144.19325 42.0205) (width 0.2) (layer "B.Cu") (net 14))
 (segment (start 115.2525 78.4225) (end 115.2525 72.86625) (width 0.2) (layer "B.Cu") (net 14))
 (segment (start 115.2525 72.86625) (end 144.19325 43.9255) (width 0.2) (layer "B.Cu") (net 14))
 (segment (start 146.33388 46.0375) (end 145.25625 46.0375) (width 0.2) (layer "F.Cu") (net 6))
 (segment (start 142.218626 54.76875) (end 147.60825 49.379126) (width 0.2) (layer "F.Cu") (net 6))
 (segment (start 138.1125 54.76875) (end 142.218626 54.76875) (width 0.2) (layer "F.Cu") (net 6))
 (segment (start 147.60825 49.379126) (end 147.60825 47.31187) (width 0.2) (layer "F.Cu") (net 6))
 (segment (start 147.60825 47.31187) (end 146.33388 46.0375) (width 0.2) (layer "F.Cu") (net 6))
 (via (at 138.1125 54.76875) (size 0.6) (drill 0.3) (layers "F.Cu" "B.Cu") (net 6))
 (segment (start 134.3025 59.3725) (end 138.1125 55.5625) (width 0.2) (layer "B.Cu") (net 6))
 (segment (start 138.1125 55.5625) (end 138.1125 54.76875) (width 0.2) (layer "B.Cu") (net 6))
 (segment (start 147.6375 65.0875) (end 147.6375 45.87875) (width 0.2) (layer "B.Cu") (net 5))
 (segment (start 147.6375 45.87875) (end 145.25625 43.4975) (width 0.2) (layer "B.Cu") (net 5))
 (segment (start 134.3025 78.4225) (end 147.6375 65.0875) (width 0.2) (layer "B.Cu") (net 5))
 (segment (start 143.7925 59.3725) (end 141.2525 61.9125) (width 0.2) (layer "F.Cu") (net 9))
 (segment (start 128.5875 61.9125) (end 126.4485 59.7735) (width 0.2) (layer "F.Cu") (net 9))
 (segment (start 153.3525 59.3725) (end 143.7925 59.3725) (width 0.2) (layer "F.Cu") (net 9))
 (segment (start 126.40525 59.7735) (end 126.20625 59.9725) (width 0.2) (layer "F.Cu") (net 9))
 (segment (start 126.4485 59.7735) (end 126.40525 59.7735) (width 0.2) (layer "F.Cu") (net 9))
 (via (at 126.20625 59.9725) (size 0.6) (drill 0.3) (layers "F.Cu" "B.Cu") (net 9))
 (via (at 128.5875 61.9125) (size 0.6) (drill 0.3) (layers "F.Cu" "B.Cu") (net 9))
 (via (at 141.2525 61.9125) (size 0.6) (drill 0.3) (layers "F.Cu" "B.Cu") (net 9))
 (segment (start 141.2525 61.9125) (end 141.2525 62.097316) (width 0.2) (layer "B.Cu") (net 9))
 (segment (start 130.9385 64.2635) (end 128.5875 61.9125) (width 0.2) (layer "B.Cu") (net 9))
 (segment (start 141.2525 62.097316) (end 139.086316 64.2635) (width 0.2) (layer "B.Cu") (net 9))
 (segment (start 139.086316 64.2635) (end 130.9385 64.2635) (width 0.2) (layer "B.Cu") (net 9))
 (segment (start 126.20625 59.9725) (end 130.01625 56.1625) (width 0.2) (layer "B.Cu") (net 9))
 (segment (start 130.01625 56.1625) (end 130.01625 48.5775) (width 0.2) (layer "B.Cu") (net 9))
 (segment (start 150.8815 41.344) (end 150.8815 75.9515) (width 0.2) (layer "B.Cu") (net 10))
 (segment (start 136.15925 39.8945) (end 149.432 39.8945) (width 0.2) (layer "B.Cu") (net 10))
 (segment (start 149.432 39.8945) (end 150.8815 41.344) (width 0.2) (layer "B.Cu") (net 10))
 (segment (start 130.01625 46.0375) (end 136.15925 39.8945) (width 0.2) (layer "B.Cu") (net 10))
 (segment (start 150.8815 75.9515) (end 153.3525 78.4225) (width 0.2) (layer "B.Cu") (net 10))
 (segment (start 112.9045 39.1795) (end 129.254251 39.179499) (width 0.2) (layer "F.Cu") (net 7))
 (segment (start 129.254251 39.179499) (end 130.01625 38.4175) (width 0.2) (layer "F.Cu") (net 7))
 (segment (start 111.70625 37.98125) (end 112.9045 39.1795) (width 0.2) (layer "F.Cu") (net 7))
 (segment (start 129.2135 36.68025) (end 110.40525 36.68025) (width 0.2) (layer "F.Cu") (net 8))
 (segment (start 110.40525 41.68025) (end 111.70625 42.98125) (width 0.2) (layer "F.Cu") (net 8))
 (segment (start 110.40525 36.68025) (end 110.40525 41.68025) (width 0.2) (layer "F.Cu") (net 8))
 (segment (start 130.01625 35.8775) (end 129.2135 36.68025) (width 0.2) (layer "F.Cu") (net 8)))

